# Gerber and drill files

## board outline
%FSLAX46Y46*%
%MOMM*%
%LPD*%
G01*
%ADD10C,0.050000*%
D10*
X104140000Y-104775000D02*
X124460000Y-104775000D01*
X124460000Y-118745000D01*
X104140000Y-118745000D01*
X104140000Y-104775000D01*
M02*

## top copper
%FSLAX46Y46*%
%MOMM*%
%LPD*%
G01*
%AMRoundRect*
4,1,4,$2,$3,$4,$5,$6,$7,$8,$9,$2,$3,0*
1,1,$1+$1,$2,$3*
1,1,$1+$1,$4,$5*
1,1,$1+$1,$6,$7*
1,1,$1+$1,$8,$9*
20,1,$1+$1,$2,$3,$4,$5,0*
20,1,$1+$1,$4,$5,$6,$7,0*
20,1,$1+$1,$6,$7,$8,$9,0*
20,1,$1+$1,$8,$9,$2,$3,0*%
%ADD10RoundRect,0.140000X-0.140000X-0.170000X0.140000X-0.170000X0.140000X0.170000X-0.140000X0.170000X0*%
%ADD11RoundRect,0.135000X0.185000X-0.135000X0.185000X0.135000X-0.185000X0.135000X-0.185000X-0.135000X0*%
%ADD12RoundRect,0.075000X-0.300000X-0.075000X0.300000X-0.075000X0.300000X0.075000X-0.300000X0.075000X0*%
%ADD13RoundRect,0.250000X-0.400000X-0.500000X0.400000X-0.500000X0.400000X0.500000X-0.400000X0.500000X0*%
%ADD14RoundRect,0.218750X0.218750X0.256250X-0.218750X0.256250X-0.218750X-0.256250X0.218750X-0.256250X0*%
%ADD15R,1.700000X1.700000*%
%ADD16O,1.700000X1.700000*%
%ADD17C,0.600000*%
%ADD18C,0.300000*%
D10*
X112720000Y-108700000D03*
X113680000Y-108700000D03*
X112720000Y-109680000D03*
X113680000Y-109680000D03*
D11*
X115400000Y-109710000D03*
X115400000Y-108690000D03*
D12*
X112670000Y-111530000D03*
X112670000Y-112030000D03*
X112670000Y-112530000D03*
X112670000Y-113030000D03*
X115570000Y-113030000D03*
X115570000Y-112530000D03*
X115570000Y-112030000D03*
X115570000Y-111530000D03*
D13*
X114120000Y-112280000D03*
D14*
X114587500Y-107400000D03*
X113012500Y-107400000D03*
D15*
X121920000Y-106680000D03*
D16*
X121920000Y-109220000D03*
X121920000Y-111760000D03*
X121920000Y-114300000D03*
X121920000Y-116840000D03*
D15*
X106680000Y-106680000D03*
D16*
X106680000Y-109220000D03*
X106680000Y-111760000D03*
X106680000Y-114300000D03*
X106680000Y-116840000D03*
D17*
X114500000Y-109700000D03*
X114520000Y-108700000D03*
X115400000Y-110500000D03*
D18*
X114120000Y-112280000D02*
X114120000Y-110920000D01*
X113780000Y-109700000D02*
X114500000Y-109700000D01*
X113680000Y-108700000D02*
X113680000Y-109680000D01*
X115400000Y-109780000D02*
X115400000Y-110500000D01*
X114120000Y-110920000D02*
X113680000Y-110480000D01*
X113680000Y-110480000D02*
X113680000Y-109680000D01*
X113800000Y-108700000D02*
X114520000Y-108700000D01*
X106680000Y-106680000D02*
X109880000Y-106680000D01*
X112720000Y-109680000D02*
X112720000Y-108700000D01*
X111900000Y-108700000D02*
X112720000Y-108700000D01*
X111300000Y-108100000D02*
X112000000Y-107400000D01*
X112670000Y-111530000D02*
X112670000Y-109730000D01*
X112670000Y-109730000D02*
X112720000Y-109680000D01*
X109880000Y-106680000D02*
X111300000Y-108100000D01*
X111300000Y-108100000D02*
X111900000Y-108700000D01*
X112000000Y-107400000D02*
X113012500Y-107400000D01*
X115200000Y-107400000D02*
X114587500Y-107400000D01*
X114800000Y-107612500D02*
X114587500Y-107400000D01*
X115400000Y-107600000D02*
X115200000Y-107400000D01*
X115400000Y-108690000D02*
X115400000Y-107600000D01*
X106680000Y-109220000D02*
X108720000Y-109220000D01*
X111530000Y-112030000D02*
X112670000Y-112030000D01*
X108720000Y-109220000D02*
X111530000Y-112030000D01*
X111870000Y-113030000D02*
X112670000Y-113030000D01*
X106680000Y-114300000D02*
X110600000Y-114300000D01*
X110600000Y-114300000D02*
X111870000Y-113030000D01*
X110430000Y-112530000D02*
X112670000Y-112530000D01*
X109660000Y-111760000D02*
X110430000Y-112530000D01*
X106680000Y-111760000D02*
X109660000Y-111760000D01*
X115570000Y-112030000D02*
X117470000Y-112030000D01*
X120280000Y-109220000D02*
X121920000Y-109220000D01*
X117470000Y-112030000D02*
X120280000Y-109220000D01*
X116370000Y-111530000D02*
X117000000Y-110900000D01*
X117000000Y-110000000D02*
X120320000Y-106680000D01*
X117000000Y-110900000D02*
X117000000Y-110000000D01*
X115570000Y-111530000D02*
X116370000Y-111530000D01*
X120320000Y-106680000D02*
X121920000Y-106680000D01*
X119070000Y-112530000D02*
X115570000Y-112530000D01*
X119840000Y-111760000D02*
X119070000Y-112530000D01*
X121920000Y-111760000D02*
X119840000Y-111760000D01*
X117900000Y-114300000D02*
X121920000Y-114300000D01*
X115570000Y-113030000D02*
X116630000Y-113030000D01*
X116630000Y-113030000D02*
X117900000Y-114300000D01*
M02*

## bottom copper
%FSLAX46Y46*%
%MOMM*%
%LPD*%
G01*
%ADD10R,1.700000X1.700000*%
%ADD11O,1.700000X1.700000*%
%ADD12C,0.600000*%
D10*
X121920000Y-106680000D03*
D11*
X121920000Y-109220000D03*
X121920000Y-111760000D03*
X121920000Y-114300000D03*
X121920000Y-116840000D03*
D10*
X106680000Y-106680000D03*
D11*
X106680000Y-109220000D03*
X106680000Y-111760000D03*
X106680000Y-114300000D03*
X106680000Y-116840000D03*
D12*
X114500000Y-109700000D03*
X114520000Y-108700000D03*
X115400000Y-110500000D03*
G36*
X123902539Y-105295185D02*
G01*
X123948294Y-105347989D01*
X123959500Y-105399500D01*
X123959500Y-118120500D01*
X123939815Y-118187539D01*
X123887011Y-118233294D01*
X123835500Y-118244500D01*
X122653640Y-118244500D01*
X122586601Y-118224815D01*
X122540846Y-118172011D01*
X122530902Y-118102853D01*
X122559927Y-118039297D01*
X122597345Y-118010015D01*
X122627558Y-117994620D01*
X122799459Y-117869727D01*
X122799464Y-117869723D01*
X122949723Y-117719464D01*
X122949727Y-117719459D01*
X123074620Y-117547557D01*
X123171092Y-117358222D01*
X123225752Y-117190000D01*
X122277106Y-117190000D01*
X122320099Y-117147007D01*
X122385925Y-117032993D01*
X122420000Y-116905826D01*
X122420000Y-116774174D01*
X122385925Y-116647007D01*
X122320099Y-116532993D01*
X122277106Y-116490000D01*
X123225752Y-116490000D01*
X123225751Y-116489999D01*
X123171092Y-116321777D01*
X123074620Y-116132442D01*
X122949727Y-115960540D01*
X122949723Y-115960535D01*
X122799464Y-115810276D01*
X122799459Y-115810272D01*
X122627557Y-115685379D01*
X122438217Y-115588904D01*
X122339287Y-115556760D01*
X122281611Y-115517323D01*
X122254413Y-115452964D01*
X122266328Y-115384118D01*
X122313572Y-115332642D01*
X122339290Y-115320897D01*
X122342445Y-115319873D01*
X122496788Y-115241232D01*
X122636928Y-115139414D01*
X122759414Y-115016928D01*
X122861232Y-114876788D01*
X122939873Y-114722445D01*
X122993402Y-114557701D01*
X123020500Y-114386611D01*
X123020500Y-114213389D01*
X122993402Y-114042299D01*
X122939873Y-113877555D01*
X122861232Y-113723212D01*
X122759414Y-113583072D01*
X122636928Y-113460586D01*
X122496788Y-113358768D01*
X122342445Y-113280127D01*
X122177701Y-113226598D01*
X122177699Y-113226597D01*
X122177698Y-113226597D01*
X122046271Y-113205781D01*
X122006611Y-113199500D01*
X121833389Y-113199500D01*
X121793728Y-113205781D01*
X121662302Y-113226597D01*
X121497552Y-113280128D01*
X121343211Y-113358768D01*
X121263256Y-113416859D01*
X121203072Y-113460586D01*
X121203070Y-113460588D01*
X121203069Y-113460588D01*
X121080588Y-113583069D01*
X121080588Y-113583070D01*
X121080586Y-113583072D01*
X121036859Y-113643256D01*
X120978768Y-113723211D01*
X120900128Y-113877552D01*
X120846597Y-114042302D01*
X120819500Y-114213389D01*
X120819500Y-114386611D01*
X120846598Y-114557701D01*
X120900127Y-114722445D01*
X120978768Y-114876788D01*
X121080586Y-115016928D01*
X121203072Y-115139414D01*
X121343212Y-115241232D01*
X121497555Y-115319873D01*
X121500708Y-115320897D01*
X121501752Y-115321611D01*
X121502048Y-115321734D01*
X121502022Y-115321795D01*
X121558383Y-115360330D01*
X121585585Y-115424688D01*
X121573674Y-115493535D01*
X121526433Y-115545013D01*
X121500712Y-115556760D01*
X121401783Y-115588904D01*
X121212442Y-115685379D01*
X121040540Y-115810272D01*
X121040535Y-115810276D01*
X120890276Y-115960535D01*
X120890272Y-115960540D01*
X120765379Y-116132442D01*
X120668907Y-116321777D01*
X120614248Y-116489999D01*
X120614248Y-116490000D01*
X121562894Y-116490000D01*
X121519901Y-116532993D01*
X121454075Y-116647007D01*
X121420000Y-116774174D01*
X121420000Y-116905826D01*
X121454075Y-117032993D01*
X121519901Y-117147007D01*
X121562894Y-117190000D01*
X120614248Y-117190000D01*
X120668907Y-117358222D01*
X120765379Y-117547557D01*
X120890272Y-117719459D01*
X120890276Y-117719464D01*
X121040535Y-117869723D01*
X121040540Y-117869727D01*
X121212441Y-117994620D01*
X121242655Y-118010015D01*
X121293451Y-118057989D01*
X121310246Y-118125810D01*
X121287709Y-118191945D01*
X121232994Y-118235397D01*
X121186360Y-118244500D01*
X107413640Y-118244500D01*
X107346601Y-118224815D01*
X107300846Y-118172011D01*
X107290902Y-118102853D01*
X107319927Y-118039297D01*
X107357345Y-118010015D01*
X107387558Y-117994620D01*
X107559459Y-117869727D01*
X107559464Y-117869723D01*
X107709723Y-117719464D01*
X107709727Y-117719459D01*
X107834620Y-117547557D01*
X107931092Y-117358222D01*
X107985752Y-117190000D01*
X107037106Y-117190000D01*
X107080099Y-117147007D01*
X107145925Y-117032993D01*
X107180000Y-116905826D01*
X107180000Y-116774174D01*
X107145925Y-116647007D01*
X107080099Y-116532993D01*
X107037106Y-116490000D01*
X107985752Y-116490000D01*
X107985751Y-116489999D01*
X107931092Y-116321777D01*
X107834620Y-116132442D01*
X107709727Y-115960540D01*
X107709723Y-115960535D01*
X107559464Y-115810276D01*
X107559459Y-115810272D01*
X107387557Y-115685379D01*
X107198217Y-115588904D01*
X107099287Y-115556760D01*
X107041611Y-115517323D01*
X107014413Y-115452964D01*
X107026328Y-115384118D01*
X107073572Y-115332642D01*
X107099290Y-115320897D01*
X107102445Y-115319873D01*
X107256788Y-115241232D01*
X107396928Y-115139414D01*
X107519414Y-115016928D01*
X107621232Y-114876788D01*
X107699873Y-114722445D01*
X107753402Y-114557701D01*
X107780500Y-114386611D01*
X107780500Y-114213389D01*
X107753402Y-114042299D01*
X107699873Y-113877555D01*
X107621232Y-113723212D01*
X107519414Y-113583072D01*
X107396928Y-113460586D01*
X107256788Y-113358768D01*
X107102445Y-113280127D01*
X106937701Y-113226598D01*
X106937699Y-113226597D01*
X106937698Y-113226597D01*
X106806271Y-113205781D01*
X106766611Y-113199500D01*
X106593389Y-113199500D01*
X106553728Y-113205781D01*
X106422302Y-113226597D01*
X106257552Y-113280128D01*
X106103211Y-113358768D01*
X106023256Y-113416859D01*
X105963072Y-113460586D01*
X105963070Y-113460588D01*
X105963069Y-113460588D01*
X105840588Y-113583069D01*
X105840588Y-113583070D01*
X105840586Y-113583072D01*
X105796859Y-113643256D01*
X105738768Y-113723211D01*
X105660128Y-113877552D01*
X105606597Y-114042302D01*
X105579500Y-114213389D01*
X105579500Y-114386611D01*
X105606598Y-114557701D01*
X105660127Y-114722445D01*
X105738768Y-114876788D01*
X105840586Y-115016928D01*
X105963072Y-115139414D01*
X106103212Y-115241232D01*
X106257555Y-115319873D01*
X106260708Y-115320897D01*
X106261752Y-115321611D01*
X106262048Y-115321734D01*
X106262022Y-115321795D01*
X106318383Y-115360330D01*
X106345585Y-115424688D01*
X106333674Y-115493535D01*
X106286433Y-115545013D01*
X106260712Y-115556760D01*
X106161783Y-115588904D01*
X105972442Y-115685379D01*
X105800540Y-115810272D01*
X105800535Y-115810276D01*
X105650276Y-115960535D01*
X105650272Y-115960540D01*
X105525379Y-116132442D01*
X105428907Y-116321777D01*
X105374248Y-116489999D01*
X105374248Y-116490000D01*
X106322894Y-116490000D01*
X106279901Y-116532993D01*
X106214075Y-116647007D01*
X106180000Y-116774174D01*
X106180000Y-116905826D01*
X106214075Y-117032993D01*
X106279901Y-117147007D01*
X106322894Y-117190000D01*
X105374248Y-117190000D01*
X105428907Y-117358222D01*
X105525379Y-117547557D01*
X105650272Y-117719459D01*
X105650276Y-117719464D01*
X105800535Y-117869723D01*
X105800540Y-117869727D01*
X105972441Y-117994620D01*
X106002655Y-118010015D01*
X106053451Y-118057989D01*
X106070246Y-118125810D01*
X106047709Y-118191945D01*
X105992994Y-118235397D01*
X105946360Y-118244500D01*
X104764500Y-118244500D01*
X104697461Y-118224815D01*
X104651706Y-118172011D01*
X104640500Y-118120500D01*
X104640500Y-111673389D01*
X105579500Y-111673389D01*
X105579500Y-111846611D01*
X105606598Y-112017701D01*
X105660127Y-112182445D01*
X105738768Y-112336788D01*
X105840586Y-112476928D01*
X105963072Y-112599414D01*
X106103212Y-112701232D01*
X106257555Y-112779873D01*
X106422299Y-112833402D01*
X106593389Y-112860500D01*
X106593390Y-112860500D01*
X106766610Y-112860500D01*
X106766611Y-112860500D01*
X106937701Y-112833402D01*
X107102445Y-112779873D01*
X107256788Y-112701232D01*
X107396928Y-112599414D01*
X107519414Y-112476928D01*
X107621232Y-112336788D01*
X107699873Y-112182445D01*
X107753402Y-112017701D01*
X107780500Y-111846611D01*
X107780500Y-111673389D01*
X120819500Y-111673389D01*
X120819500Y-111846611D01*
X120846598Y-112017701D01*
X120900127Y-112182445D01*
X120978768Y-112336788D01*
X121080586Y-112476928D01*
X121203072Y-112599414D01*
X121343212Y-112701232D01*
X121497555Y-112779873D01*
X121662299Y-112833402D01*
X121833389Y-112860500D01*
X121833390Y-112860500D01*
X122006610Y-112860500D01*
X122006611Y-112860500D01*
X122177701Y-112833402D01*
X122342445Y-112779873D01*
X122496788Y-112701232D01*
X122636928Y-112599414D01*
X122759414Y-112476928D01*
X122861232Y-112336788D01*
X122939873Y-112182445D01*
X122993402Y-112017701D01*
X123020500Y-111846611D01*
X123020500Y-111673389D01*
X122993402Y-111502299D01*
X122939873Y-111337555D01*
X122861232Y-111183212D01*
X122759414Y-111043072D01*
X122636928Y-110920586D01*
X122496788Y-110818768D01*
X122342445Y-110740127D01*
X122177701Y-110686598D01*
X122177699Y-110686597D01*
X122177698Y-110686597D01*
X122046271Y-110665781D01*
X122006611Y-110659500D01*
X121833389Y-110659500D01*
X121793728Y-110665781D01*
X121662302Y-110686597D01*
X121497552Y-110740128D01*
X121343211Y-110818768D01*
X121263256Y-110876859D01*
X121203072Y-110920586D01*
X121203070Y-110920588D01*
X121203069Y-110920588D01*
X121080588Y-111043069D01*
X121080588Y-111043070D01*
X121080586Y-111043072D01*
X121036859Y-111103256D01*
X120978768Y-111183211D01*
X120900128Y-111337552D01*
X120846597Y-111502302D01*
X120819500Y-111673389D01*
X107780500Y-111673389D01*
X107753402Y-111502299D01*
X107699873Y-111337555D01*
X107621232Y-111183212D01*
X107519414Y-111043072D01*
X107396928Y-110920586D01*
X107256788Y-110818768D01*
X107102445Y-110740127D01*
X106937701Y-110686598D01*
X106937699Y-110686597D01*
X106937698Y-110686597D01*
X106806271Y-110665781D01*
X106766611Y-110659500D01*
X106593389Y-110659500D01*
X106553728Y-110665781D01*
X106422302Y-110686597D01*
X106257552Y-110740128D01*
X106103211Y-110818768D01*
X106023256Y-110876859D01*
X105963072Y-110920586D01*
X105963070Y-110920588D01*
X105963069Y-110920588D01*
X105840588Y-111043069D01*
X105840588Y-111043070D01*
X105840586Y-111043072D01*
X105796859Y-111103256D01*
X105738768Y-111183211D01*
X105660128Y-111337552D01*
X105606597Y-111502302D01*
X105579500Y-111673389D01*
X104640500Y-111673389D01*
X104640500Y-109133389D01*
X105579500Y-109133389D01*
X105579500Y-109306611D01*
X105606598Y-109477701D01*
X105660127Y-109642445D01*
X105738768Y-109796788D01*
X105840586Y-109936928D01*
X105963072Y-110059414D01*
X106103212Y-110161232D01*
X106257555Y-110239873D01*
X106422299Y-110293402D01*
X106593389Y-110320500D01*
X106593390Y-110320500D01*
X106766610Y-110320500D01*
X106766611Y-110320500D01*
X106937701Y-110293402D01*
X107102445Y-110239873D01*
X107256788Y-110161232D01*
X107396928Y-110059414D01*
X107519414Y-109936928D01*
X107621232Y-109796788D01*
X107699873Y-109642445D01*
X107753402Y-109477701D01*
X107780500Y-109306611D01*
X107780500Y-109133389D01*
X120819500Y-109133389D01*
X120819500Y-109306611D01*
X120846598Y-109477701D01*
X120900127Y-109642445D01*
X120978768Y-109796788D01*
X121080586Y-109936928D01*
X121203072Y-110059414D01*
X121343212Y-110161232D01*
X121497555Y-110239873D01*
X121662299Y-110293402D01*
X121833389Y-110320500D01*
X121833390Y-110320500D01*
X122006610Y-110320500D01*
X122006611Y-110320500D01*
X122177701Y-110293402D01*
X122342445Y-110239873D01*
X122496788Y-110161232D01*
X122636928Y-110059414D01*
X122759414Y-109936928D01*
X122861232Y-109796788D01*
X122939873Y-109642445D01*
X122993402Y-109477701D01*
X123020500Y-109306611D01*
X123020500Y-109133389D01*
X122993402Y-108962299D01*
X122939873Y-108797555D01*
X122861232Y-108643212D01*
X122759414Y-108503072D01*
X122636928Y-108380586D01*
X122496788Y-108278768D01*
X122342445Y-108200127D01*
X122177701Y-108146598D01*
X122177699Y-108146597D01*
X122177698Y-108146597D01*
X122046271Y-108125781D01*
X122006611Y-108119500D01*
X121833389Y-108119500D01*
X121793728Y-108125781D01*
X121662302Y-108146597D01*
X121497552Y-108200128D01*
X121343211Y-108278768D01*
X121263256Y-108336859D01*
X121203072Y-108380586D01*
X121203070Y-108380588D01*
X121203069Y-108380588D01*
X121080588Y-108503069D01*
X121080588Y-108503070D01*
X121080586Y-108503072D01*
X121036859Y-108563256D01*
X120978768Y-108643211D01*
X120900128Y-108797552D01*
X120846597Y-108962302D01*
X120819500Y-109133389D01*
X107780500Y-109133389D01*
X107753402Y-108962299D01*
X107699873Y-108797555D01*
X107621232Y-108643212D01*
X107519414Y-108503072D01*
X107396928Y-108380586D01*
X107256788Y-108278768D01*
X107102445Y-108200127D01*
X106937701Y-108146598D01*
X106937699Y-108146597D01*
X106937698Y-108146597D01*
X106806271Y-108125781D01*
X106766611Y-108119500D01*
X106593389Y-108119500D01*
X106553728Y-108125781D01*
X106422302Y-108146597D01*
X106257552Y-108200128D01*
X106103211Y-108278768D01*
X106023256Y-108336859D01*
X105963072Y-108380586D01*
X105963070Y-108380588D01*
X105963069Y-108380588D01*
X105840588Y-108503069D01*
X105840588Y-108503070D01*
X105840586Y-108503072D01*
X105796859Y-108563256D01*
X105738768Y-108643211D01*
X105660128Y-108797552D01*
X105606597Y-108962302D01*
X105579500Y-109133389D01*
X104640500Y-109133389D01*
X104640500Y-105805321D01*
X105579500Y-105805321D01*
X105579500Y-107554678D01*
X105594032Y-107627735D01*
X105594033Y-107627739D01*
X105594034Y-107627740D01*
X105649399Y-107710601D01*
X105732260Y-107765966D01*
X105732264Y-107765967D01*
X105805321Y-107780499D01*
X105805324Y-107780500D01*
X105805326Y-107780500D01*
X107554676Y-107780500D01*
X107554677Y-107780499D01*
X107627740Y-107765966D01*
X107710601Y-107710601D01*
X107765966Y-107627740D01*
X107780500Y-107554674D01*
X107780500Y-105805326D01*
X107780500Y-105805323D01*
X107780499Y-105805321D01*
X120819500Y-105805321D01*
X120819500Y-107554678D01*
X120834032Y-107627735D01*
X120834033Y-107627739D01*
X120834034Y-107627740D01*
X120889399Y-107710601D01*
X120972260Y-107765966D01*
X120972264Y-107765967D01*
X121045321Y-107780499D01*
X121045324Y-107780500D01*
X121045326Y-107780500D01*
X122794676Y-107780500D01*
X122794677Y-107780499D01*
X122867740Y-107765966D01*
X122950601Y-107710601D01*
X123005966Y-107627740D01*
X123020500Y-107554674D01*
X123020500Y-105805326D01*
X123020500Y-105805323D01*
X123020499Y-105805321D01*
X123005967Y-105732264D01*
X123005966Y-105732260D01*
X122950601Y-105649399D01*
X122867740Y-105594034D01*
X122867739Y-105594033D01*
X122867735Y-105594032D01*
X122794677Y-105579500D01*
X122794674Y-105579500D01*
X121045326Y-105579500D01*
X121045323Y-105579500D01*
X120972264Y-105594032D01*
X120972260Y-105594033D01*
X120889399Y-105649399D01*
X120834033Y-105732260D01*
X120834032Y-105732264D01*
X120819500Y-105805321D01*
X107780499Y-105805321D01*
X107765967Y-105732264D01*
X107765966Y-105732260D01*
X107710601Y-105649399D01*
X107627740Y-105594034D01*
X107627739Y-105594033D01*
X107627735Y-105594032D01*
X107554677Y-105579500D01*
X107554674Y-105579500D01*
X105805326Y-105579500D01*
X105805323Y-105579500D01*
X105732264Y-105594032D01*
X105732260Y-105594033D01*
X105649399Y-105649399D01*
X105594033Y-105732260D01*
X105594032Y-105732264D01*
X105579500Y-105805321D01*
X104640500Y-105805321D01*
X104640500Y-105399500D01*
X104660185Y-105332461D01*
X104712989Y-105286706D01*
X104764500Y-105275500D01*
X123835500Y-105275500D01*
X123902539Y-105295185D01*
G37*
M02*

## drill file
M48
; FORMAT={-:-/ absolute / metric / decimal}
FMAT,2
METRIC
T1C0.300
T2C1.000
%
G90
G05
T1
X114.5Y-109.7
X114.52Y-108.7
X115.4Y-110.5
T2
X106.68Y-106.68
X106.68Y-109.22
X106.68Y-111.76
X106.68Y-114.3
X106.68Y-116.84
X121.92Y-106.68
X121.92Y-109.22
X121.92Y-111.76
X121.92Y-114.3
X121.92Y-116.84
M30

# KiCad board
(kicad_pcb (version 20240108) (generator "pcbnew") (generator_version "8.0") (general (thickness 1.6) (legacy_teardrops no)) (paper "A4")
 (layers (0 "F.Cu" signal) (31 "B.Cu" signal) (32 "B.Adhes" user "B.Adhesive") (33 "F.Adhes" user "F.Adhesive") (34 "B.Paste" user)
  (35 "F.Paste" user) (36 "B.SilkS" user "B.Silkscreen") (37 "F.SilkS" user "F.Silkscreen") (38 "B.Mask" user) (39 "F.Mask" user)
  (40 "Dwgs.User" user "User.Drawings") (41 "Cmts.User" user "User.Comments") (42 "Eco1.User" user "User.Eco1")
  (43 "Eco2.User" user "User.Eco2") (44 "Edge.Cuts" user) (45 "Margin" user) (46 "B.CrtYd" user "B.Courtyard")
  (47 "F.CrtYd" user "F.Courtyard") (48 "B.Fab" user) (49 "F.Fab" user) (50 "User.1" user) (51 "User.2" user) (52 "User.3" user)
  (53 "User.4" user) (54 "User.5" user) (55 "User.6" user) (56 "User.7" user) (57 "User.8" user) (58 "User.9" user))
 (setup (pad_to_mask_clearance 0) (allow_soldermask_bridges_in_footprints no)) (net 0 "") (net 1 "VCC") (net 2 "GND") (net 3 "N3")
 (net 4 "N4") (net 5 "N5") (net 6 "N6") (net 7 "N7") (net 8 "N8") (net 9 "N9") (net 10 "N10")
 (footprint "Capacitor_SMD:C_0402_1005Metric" (layer "F.Cu") (at 113.2 108.7)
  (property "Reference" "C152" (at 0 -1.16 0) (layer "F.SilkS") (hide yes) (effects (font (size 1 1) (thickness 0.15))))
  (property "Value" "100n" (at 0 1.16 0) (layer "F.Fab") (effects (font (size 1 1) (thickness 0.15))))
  (pad "1" smd roundrect (at -0.48 0) (size 0.56 0.62) (layers "F.Cu" "F.Paste" "F.Mask") (roundrect_rratio 0.25) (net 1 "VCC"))
  (pad "2" smd roundrect (at 0.48 0) (size 0.56 0.62) (layers "F.Cu" "F.Paste" "F.Mask") (roundrect_rratio 0.25) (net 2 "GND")))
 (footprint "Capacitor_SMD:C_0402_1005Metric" (layer "F.Cu") (at 113.2 109.68)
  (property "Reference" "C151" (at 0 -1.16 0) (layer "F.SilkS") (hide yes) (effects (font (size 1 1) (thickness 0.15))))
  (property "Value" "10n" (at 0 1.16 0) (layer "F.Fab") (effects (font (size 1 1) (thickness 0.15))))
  (pad "1" smd roundrect (at -0.48 0) (size 0.56 0.62) (layers "F.Cu" "F.Paste" "F.Mask") (roundrect_rratio 0.25) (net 1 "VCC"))
  (pad "2" smd roundrect (at 0.48 0) (size 0.56 0.62) (layers "F.Cu" "F.Paste" "F.Mask") (roundrect_rratio 0.25) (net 2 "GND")))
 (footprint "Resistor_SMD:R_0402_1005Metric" (layer "F.Cu") (at 115.4 109.2 90)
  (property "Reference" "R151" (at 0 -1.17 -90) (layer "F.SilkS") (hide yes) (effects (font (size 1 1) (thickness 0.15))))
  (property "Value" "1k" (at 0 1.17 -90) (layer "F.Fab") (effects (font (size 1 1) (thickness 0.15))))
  (pad "1" smd roundrect (at -0.51 0 90) (size 0.54 0.64) (layers "F.Cu" "F.Paste" "F.Mask") (roundrect_rratio 0.25) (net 2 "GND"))
  (pad "2" smd roundrect (at 0.51 0 90) (size 0.54 0.64) (layers "F.Cu" "F.Paste" "F.Mask") (roundrect_rratio 0.25) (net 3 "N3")))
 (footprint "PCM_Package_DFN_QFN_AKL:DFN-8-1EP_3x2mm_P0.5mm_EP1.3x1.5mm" (layer "F.Cu") (at 114.12 112.28)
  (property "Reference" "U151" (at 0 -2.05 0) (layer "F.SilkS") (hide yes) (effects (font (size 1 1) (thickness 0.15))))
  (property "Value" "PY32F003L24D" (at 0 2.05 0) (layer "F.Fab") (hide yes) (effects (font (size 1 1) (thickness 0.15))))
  (pad "" smd roundrect (at -0.325 -0.375) (size 0.5 0.6) (layers "F.Paste") (roundrect_rratio 0.25))
  (pad "" smd roundrect (at -0.325 0.375) (size 0.5 0.6) (layers "F.Paste") (roundrect_rratio 0.25))
  (pad "" smd roundrect (at 0.325 -0.375) (size 0.5 0.6) (layers "F.Paste") (roundrect_rratio 0.25))
  (pad "" smd roundrect (at 0.325 0.375) (size 0.5 0.6) (layers "F.Paste") (roundrect_rratio 0.25))
  (pad "1" smd roundrect (at -1.45 -0.75) (size 0.75 0.3) (layers "F.Cu" "F.Paste" "F.Mask") (roundrect_rratio 0.25) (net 1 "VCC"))
  (pad "2" smd roundrect (at -1.45 -0.25) (size 0.75 0.3) (layers "F.Cu" "F.Paste" "F.Mask") (roundrect_rratio 0.25) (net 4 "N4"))
  (pad "3" smd roundrect (at -1.45 0.25) (size 0.75 0.3) (layers "F.Cu" "F.Paste" "F.Mask") (roundrect_rratio 0.25) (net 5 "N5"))
  (pad "4" smd roundrect (at -1.45 0.75) (size 0.75 0.3) (layers "F.Cu" "F.Paste" "F.Mask") (roundrect_rratio 0.25) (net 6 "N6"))
  (pad "5" smd roundrect (at 1.45 0.75) (size 0.75 0.3) (layers "F.Cu" "F.Paste" "F.Mask") (roundrect_rratio 0.25) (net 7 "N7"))
  (pad "6" smd roundrect (at 1.45 0.25) (size 0.75 0.3) (layers "F.Cu" "F.Paste" "F.Mask") (roundrect_rratio 0.25) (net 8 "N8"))
  (pad "7" smd roundrect (at 1.45 -0.25) (size 0.75 0.3) (layers "F.Cu" "F.Paste" "F.Mask") (roundrect_rratio 0.25) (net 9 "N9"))
  (pad "8" smd roundrect (at 1.45 -0.75) (size 0.75 0.3) (layers "F.Cu" "F.Paste" "F.Mask") (roundrect_rratio 0.25) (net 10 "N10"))
  (pad "9" smd roundrect (at 0 0) (size 1.3 1.5) (layers "F.Cu" "F.Mask") (roundrect_rratio 0.1923076923) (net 2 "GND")))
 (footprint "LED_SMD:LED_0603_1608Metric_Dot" (layer "F.Cu") (at 113.8 107.4 180)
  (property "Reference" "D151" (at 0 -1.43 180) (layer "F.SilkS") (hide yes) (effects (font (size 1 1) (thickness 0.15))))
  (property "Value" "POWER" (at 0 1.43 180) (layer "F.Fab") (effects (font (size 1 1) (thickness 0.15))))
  (pad "1" smd roundrect (at -0.7875 0 180) (size 0.875 0.95) (layers "F.Cu" "F.Paste" "F.Mask") (roundrect_rratio 0.25) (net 3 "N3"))
  (pad "2" smd roundrect (at 0.7875 0 180) (size 0.875 0.95) (layers "F.Cu" "F.Paste" "F.Mask") (roundrect_rratio 0.25) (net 1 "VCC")))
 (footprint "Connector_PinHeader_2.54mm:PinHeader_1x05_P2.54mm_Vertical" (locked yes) (layer "B.Cu") (at 121.92 106.68 180)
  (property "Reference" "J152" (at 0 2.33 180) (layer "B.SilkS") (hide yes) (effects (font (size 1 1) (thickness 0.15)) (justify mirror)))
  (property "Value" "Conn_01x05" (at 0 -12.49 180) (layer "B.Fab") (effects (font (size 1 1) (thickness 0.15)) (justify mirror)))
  (pad "1" thru_hole rect (at 0 0 180) (size 1.7 1.7) (drill 1) (layers "*.Cu" "*.Mask") (remove_unused_layers no) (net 10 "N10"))
  (pad "2" thru_hole oval (at 0 -2.54 180) (size 1.7 1.7) (drill 1) (layers "*.Cu" "*.Mask") (remove_unused_layers no) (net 9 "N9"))
  (pad "3" thru_hole oval (at 0 -5.08 180) (size 1.7 1.7) (drill 1) (layers "*.Cu" "*.Mask") (remove_unused_layers no) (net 8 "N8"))
  (pad "4" thru_hole oval (at 0 -7.62 180) (size 1.7 1.7) (drill 1) (layers "*.Cu" "*.Mask") (remove_unused_layers no) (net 7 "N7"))
  (pad "5" thru_hole oval (at 0 -10.16 180) (size 1.7 1.7) (drill 1) (layers "*.Cu" "*.Mask") (remove_unused_layers no) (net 2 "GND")))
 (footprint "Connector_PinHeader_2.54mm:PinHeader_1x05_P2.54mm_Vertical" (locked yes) (layer "B.Cu") (at 106.68 106.68 180)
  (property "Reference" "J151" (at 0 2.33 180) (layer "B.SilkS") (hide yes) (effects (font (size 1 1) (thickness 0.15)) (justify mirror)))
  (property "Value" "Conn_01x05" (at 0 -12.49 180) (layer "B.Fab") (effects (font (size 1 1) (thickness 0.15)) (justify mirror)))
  (pad "1" thru_hole rect (at 0 0 180) (size 1.7 1.7) (drill 1) (layers "*.Cu" "*.Mask") (remove_unused_layers no) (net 1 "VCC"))
  (pad "2" thru_hole oval (at 0 -2.54 180) (size 1.7 1.7) (drill 1) (layers "*.Cu" "*.Mask") (remove_unused_layers no) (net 4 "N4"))
  (pad "3" thru_hole oval (at 0 -5.08 180) (size 1.7 1.7) (drill 1) (layers "*.Cu" "*.Mask") (remove_unused_layers no) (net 5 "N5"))
  (pad "4" thru_hole oval (at 0 -7.62 180) (size 1.7 1.7) (drill 1) (layers "*.Cu" "*.Mask") (remove_unused_layers no) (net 6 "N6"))
  (pad "5" thru_hole oval (at 0 -10.16 180) (size 1.7 1.7) (drill 1) (layers "*.Cu" "*.Mask") (remove_unused_layers no) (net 2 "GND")))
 (gr_rect (start 104.14 104.775) (end 124.46 118.745) (stroke (width 0.05) (type default)) (fill none) (layer "Edge.Cuts"))
 (segment (start 114.12 112.28) (end 114.12 110.92) (width 0.3) (layer "F.Cu") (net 2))
 (segment (start 113.78 109.7) (end 114.5 109.7) (width 0.3) (layer "F.Cu") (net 2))
 (segment (start 113.68 108.7) (end 113.68 109.68) (width 0.3) (layer "F.Cu") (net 2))
 (segment (start 115.4 109.78) (end 115.4 110.5) (width 0.3) (layer "F.Cu") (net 2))
 (segment (start 114.12 110.92) (end 113.68 110.48) (width 0.3) (layer "F.Cu") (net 2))
 (segment (start 113.68 110.48) (end 113.68 109.68) (width 0.3) (layer "F.Cu") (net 2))
 (segment (start 113.8 108.7) (end 114.52 108.7) (width 0.3) (layer "F.Cu") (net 2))
 (via (at 114.5 109.7) (size 0.6) (drill 0.3) (layers "F.Cu" "B.Cu") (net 2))
 (via (at 114.52 108.7) (size 0.6) (drill 0.3) (layers "F.Cu" "B.Cu") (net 2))
 (via (at 115.4 110.5) (size 0.6) (drill 0.3) (layers "F.Cu" "B.Cu") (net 2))
 (segment (start 106.68 106.68) (end 109.88 106.68) (width 0.3) (layer "F.Cu") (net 1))
 (segment (start 112.72 109.68) (end 112.72 108.7) (width 0.3) (layer "F.Cu") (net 1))
 (segment (start 111.9 108.7) (end 112.72 108.7) (width 0.3) (layer "F.Cu") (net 1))
 (segment (start 111.3 108.1) (end 112 107.4) (width 0.3) (layer "F.Cu") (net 1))
 (segment (start 112.67 111.53) (end 112.67 109.73) (width 0.3) (layer "F.Cu") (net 1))
 (segment (start 112.67 109.73) (end 112.72 109.68) (width 0.3) (layer "F.Cu") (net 1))
 (segment (start 109.88 106.68) (end 111.3 108.1) (width 0.3) (layer "F.Cu") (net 1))
 (segment (start 111.3 108.1) (end 111.9 108.7) (width 0.3) (layer "F.Cu") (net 1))
 (segment (start 112 107.4) (end 113.0125 107.4) (width 0.3) (layer "F.Cu") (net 1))
 (segment (start 115.2 107.4) (end 114.5875 107.4) (width 0.3) (layer "F.Cu") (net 3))
 (segment (start 114.8 107.6125) (end 114.5875 107.4) (width 0.3) (layer "F.Cu") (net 3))
 (segment (start 115.4 107.6) (end 115.2 107.4) (width 0.3) (layer "F.Cu") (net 3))
 (segment (start 115.4 108.69) (end 115.4 107.6) (width 0.3) (layer "F.Cu") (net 3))
 (segment (start 106.68 109.22) (end 108.72 109.22) (width 0.3) (layer "F.Cu") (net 4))
 (segment (start 111.53 112.03) (end 112.67 112.03) (width 0.3) (layer "F.Cu") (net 4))
 (segment (start 108.72 109.22) (end 111.53 112.03) (width 0.3) (layer "F.Cu") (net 4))
 (segment (start 111.87 113.03) (end 112.67 113.03) (width 0.3) (layer "F.Cu") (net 6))
 (segment (start 106.68 114.3) (end 110.6 114.3) (width 0.3) (layer "F.Cu") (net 6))
 (segment (start 110.6 114.3) (end 111.87 113.03) (width 0.3) (layer "F.Cu") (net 6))
 (segment (start 110.43 112.53) (end 112.67 112.53) (width 0.3) (layer "F.Cu") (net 5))
 (segment (start 109.66 111.76) (end 110.43 112.53) (width 0.3) (layer "F.Cu") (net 5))
 (segment (start 106.68 111.76) (end 109.66 111.76) (width 0.3) (layer "F.Cu") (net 5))
 (segment (start 115.57 112.03) (end 117.47 112.03) (width 0.3) (layer "F.Cu") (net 9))
 (segment (start 120.28 109.22) (end 121.92 109.22) (width 0.3) (layer "F.Cu") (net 9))
 (segment (start 117.47 112.03) (end 120.28 109.22) (width 0.3) (layer "F.Cu") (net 9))
 (segment (start 116.37 111.53) (end 117 110.9) (width 0.3) (layer "F.Cu") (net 10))
 (segment (start 117 110) (end 120.32 106.68) (width 0.3) (layer "F.Cu") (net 10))
 (segment (start 117 110.9) (end 117 110) (width 0.3) (layer "F.Cu") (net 10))
 (segment (start 115.57 111.53) (end 116.37 111.53) (width 0.3) (layer "F.Cu") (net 10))
 (segment (start 120.32 106.68) (end 121.92 106.68) (width 0.3) (layer "F.Cu") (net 10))
 (segment (start 119.07 112.53) (end 115.57 112.53) (width 0.3) (layer "F.Cu") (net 8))
 (segment (start 119.84 111.76) (end 119.07 112.53) (width 0.3) (layer "F.Cu") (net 8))
 (segment (start 121.92 111.76) (end 119.84 111.76) (width 0.3) (layer "F.Cu") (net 8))
 (segment (start 117.9 114.3) (end 121.92 114.3) (width 0.3) (layer "F.Cu") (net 7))
 (segment (start 115.57 113.03) (end 116.63 113.03) (width 0.3) (layer "F.Cu") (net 7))
 (segment (start 116.63 113.03) (end 117.9 114.3) (width 0.3) (layer "F.Cu") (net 7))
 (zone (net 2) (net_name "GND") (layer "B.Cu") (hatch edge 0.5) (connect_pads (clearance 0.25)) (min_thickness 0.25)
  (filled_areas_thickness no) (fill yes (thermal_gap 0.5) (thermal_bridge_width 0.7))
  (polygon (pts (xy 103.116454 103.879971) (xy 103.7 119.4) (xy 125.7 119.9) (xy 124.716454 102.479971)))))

